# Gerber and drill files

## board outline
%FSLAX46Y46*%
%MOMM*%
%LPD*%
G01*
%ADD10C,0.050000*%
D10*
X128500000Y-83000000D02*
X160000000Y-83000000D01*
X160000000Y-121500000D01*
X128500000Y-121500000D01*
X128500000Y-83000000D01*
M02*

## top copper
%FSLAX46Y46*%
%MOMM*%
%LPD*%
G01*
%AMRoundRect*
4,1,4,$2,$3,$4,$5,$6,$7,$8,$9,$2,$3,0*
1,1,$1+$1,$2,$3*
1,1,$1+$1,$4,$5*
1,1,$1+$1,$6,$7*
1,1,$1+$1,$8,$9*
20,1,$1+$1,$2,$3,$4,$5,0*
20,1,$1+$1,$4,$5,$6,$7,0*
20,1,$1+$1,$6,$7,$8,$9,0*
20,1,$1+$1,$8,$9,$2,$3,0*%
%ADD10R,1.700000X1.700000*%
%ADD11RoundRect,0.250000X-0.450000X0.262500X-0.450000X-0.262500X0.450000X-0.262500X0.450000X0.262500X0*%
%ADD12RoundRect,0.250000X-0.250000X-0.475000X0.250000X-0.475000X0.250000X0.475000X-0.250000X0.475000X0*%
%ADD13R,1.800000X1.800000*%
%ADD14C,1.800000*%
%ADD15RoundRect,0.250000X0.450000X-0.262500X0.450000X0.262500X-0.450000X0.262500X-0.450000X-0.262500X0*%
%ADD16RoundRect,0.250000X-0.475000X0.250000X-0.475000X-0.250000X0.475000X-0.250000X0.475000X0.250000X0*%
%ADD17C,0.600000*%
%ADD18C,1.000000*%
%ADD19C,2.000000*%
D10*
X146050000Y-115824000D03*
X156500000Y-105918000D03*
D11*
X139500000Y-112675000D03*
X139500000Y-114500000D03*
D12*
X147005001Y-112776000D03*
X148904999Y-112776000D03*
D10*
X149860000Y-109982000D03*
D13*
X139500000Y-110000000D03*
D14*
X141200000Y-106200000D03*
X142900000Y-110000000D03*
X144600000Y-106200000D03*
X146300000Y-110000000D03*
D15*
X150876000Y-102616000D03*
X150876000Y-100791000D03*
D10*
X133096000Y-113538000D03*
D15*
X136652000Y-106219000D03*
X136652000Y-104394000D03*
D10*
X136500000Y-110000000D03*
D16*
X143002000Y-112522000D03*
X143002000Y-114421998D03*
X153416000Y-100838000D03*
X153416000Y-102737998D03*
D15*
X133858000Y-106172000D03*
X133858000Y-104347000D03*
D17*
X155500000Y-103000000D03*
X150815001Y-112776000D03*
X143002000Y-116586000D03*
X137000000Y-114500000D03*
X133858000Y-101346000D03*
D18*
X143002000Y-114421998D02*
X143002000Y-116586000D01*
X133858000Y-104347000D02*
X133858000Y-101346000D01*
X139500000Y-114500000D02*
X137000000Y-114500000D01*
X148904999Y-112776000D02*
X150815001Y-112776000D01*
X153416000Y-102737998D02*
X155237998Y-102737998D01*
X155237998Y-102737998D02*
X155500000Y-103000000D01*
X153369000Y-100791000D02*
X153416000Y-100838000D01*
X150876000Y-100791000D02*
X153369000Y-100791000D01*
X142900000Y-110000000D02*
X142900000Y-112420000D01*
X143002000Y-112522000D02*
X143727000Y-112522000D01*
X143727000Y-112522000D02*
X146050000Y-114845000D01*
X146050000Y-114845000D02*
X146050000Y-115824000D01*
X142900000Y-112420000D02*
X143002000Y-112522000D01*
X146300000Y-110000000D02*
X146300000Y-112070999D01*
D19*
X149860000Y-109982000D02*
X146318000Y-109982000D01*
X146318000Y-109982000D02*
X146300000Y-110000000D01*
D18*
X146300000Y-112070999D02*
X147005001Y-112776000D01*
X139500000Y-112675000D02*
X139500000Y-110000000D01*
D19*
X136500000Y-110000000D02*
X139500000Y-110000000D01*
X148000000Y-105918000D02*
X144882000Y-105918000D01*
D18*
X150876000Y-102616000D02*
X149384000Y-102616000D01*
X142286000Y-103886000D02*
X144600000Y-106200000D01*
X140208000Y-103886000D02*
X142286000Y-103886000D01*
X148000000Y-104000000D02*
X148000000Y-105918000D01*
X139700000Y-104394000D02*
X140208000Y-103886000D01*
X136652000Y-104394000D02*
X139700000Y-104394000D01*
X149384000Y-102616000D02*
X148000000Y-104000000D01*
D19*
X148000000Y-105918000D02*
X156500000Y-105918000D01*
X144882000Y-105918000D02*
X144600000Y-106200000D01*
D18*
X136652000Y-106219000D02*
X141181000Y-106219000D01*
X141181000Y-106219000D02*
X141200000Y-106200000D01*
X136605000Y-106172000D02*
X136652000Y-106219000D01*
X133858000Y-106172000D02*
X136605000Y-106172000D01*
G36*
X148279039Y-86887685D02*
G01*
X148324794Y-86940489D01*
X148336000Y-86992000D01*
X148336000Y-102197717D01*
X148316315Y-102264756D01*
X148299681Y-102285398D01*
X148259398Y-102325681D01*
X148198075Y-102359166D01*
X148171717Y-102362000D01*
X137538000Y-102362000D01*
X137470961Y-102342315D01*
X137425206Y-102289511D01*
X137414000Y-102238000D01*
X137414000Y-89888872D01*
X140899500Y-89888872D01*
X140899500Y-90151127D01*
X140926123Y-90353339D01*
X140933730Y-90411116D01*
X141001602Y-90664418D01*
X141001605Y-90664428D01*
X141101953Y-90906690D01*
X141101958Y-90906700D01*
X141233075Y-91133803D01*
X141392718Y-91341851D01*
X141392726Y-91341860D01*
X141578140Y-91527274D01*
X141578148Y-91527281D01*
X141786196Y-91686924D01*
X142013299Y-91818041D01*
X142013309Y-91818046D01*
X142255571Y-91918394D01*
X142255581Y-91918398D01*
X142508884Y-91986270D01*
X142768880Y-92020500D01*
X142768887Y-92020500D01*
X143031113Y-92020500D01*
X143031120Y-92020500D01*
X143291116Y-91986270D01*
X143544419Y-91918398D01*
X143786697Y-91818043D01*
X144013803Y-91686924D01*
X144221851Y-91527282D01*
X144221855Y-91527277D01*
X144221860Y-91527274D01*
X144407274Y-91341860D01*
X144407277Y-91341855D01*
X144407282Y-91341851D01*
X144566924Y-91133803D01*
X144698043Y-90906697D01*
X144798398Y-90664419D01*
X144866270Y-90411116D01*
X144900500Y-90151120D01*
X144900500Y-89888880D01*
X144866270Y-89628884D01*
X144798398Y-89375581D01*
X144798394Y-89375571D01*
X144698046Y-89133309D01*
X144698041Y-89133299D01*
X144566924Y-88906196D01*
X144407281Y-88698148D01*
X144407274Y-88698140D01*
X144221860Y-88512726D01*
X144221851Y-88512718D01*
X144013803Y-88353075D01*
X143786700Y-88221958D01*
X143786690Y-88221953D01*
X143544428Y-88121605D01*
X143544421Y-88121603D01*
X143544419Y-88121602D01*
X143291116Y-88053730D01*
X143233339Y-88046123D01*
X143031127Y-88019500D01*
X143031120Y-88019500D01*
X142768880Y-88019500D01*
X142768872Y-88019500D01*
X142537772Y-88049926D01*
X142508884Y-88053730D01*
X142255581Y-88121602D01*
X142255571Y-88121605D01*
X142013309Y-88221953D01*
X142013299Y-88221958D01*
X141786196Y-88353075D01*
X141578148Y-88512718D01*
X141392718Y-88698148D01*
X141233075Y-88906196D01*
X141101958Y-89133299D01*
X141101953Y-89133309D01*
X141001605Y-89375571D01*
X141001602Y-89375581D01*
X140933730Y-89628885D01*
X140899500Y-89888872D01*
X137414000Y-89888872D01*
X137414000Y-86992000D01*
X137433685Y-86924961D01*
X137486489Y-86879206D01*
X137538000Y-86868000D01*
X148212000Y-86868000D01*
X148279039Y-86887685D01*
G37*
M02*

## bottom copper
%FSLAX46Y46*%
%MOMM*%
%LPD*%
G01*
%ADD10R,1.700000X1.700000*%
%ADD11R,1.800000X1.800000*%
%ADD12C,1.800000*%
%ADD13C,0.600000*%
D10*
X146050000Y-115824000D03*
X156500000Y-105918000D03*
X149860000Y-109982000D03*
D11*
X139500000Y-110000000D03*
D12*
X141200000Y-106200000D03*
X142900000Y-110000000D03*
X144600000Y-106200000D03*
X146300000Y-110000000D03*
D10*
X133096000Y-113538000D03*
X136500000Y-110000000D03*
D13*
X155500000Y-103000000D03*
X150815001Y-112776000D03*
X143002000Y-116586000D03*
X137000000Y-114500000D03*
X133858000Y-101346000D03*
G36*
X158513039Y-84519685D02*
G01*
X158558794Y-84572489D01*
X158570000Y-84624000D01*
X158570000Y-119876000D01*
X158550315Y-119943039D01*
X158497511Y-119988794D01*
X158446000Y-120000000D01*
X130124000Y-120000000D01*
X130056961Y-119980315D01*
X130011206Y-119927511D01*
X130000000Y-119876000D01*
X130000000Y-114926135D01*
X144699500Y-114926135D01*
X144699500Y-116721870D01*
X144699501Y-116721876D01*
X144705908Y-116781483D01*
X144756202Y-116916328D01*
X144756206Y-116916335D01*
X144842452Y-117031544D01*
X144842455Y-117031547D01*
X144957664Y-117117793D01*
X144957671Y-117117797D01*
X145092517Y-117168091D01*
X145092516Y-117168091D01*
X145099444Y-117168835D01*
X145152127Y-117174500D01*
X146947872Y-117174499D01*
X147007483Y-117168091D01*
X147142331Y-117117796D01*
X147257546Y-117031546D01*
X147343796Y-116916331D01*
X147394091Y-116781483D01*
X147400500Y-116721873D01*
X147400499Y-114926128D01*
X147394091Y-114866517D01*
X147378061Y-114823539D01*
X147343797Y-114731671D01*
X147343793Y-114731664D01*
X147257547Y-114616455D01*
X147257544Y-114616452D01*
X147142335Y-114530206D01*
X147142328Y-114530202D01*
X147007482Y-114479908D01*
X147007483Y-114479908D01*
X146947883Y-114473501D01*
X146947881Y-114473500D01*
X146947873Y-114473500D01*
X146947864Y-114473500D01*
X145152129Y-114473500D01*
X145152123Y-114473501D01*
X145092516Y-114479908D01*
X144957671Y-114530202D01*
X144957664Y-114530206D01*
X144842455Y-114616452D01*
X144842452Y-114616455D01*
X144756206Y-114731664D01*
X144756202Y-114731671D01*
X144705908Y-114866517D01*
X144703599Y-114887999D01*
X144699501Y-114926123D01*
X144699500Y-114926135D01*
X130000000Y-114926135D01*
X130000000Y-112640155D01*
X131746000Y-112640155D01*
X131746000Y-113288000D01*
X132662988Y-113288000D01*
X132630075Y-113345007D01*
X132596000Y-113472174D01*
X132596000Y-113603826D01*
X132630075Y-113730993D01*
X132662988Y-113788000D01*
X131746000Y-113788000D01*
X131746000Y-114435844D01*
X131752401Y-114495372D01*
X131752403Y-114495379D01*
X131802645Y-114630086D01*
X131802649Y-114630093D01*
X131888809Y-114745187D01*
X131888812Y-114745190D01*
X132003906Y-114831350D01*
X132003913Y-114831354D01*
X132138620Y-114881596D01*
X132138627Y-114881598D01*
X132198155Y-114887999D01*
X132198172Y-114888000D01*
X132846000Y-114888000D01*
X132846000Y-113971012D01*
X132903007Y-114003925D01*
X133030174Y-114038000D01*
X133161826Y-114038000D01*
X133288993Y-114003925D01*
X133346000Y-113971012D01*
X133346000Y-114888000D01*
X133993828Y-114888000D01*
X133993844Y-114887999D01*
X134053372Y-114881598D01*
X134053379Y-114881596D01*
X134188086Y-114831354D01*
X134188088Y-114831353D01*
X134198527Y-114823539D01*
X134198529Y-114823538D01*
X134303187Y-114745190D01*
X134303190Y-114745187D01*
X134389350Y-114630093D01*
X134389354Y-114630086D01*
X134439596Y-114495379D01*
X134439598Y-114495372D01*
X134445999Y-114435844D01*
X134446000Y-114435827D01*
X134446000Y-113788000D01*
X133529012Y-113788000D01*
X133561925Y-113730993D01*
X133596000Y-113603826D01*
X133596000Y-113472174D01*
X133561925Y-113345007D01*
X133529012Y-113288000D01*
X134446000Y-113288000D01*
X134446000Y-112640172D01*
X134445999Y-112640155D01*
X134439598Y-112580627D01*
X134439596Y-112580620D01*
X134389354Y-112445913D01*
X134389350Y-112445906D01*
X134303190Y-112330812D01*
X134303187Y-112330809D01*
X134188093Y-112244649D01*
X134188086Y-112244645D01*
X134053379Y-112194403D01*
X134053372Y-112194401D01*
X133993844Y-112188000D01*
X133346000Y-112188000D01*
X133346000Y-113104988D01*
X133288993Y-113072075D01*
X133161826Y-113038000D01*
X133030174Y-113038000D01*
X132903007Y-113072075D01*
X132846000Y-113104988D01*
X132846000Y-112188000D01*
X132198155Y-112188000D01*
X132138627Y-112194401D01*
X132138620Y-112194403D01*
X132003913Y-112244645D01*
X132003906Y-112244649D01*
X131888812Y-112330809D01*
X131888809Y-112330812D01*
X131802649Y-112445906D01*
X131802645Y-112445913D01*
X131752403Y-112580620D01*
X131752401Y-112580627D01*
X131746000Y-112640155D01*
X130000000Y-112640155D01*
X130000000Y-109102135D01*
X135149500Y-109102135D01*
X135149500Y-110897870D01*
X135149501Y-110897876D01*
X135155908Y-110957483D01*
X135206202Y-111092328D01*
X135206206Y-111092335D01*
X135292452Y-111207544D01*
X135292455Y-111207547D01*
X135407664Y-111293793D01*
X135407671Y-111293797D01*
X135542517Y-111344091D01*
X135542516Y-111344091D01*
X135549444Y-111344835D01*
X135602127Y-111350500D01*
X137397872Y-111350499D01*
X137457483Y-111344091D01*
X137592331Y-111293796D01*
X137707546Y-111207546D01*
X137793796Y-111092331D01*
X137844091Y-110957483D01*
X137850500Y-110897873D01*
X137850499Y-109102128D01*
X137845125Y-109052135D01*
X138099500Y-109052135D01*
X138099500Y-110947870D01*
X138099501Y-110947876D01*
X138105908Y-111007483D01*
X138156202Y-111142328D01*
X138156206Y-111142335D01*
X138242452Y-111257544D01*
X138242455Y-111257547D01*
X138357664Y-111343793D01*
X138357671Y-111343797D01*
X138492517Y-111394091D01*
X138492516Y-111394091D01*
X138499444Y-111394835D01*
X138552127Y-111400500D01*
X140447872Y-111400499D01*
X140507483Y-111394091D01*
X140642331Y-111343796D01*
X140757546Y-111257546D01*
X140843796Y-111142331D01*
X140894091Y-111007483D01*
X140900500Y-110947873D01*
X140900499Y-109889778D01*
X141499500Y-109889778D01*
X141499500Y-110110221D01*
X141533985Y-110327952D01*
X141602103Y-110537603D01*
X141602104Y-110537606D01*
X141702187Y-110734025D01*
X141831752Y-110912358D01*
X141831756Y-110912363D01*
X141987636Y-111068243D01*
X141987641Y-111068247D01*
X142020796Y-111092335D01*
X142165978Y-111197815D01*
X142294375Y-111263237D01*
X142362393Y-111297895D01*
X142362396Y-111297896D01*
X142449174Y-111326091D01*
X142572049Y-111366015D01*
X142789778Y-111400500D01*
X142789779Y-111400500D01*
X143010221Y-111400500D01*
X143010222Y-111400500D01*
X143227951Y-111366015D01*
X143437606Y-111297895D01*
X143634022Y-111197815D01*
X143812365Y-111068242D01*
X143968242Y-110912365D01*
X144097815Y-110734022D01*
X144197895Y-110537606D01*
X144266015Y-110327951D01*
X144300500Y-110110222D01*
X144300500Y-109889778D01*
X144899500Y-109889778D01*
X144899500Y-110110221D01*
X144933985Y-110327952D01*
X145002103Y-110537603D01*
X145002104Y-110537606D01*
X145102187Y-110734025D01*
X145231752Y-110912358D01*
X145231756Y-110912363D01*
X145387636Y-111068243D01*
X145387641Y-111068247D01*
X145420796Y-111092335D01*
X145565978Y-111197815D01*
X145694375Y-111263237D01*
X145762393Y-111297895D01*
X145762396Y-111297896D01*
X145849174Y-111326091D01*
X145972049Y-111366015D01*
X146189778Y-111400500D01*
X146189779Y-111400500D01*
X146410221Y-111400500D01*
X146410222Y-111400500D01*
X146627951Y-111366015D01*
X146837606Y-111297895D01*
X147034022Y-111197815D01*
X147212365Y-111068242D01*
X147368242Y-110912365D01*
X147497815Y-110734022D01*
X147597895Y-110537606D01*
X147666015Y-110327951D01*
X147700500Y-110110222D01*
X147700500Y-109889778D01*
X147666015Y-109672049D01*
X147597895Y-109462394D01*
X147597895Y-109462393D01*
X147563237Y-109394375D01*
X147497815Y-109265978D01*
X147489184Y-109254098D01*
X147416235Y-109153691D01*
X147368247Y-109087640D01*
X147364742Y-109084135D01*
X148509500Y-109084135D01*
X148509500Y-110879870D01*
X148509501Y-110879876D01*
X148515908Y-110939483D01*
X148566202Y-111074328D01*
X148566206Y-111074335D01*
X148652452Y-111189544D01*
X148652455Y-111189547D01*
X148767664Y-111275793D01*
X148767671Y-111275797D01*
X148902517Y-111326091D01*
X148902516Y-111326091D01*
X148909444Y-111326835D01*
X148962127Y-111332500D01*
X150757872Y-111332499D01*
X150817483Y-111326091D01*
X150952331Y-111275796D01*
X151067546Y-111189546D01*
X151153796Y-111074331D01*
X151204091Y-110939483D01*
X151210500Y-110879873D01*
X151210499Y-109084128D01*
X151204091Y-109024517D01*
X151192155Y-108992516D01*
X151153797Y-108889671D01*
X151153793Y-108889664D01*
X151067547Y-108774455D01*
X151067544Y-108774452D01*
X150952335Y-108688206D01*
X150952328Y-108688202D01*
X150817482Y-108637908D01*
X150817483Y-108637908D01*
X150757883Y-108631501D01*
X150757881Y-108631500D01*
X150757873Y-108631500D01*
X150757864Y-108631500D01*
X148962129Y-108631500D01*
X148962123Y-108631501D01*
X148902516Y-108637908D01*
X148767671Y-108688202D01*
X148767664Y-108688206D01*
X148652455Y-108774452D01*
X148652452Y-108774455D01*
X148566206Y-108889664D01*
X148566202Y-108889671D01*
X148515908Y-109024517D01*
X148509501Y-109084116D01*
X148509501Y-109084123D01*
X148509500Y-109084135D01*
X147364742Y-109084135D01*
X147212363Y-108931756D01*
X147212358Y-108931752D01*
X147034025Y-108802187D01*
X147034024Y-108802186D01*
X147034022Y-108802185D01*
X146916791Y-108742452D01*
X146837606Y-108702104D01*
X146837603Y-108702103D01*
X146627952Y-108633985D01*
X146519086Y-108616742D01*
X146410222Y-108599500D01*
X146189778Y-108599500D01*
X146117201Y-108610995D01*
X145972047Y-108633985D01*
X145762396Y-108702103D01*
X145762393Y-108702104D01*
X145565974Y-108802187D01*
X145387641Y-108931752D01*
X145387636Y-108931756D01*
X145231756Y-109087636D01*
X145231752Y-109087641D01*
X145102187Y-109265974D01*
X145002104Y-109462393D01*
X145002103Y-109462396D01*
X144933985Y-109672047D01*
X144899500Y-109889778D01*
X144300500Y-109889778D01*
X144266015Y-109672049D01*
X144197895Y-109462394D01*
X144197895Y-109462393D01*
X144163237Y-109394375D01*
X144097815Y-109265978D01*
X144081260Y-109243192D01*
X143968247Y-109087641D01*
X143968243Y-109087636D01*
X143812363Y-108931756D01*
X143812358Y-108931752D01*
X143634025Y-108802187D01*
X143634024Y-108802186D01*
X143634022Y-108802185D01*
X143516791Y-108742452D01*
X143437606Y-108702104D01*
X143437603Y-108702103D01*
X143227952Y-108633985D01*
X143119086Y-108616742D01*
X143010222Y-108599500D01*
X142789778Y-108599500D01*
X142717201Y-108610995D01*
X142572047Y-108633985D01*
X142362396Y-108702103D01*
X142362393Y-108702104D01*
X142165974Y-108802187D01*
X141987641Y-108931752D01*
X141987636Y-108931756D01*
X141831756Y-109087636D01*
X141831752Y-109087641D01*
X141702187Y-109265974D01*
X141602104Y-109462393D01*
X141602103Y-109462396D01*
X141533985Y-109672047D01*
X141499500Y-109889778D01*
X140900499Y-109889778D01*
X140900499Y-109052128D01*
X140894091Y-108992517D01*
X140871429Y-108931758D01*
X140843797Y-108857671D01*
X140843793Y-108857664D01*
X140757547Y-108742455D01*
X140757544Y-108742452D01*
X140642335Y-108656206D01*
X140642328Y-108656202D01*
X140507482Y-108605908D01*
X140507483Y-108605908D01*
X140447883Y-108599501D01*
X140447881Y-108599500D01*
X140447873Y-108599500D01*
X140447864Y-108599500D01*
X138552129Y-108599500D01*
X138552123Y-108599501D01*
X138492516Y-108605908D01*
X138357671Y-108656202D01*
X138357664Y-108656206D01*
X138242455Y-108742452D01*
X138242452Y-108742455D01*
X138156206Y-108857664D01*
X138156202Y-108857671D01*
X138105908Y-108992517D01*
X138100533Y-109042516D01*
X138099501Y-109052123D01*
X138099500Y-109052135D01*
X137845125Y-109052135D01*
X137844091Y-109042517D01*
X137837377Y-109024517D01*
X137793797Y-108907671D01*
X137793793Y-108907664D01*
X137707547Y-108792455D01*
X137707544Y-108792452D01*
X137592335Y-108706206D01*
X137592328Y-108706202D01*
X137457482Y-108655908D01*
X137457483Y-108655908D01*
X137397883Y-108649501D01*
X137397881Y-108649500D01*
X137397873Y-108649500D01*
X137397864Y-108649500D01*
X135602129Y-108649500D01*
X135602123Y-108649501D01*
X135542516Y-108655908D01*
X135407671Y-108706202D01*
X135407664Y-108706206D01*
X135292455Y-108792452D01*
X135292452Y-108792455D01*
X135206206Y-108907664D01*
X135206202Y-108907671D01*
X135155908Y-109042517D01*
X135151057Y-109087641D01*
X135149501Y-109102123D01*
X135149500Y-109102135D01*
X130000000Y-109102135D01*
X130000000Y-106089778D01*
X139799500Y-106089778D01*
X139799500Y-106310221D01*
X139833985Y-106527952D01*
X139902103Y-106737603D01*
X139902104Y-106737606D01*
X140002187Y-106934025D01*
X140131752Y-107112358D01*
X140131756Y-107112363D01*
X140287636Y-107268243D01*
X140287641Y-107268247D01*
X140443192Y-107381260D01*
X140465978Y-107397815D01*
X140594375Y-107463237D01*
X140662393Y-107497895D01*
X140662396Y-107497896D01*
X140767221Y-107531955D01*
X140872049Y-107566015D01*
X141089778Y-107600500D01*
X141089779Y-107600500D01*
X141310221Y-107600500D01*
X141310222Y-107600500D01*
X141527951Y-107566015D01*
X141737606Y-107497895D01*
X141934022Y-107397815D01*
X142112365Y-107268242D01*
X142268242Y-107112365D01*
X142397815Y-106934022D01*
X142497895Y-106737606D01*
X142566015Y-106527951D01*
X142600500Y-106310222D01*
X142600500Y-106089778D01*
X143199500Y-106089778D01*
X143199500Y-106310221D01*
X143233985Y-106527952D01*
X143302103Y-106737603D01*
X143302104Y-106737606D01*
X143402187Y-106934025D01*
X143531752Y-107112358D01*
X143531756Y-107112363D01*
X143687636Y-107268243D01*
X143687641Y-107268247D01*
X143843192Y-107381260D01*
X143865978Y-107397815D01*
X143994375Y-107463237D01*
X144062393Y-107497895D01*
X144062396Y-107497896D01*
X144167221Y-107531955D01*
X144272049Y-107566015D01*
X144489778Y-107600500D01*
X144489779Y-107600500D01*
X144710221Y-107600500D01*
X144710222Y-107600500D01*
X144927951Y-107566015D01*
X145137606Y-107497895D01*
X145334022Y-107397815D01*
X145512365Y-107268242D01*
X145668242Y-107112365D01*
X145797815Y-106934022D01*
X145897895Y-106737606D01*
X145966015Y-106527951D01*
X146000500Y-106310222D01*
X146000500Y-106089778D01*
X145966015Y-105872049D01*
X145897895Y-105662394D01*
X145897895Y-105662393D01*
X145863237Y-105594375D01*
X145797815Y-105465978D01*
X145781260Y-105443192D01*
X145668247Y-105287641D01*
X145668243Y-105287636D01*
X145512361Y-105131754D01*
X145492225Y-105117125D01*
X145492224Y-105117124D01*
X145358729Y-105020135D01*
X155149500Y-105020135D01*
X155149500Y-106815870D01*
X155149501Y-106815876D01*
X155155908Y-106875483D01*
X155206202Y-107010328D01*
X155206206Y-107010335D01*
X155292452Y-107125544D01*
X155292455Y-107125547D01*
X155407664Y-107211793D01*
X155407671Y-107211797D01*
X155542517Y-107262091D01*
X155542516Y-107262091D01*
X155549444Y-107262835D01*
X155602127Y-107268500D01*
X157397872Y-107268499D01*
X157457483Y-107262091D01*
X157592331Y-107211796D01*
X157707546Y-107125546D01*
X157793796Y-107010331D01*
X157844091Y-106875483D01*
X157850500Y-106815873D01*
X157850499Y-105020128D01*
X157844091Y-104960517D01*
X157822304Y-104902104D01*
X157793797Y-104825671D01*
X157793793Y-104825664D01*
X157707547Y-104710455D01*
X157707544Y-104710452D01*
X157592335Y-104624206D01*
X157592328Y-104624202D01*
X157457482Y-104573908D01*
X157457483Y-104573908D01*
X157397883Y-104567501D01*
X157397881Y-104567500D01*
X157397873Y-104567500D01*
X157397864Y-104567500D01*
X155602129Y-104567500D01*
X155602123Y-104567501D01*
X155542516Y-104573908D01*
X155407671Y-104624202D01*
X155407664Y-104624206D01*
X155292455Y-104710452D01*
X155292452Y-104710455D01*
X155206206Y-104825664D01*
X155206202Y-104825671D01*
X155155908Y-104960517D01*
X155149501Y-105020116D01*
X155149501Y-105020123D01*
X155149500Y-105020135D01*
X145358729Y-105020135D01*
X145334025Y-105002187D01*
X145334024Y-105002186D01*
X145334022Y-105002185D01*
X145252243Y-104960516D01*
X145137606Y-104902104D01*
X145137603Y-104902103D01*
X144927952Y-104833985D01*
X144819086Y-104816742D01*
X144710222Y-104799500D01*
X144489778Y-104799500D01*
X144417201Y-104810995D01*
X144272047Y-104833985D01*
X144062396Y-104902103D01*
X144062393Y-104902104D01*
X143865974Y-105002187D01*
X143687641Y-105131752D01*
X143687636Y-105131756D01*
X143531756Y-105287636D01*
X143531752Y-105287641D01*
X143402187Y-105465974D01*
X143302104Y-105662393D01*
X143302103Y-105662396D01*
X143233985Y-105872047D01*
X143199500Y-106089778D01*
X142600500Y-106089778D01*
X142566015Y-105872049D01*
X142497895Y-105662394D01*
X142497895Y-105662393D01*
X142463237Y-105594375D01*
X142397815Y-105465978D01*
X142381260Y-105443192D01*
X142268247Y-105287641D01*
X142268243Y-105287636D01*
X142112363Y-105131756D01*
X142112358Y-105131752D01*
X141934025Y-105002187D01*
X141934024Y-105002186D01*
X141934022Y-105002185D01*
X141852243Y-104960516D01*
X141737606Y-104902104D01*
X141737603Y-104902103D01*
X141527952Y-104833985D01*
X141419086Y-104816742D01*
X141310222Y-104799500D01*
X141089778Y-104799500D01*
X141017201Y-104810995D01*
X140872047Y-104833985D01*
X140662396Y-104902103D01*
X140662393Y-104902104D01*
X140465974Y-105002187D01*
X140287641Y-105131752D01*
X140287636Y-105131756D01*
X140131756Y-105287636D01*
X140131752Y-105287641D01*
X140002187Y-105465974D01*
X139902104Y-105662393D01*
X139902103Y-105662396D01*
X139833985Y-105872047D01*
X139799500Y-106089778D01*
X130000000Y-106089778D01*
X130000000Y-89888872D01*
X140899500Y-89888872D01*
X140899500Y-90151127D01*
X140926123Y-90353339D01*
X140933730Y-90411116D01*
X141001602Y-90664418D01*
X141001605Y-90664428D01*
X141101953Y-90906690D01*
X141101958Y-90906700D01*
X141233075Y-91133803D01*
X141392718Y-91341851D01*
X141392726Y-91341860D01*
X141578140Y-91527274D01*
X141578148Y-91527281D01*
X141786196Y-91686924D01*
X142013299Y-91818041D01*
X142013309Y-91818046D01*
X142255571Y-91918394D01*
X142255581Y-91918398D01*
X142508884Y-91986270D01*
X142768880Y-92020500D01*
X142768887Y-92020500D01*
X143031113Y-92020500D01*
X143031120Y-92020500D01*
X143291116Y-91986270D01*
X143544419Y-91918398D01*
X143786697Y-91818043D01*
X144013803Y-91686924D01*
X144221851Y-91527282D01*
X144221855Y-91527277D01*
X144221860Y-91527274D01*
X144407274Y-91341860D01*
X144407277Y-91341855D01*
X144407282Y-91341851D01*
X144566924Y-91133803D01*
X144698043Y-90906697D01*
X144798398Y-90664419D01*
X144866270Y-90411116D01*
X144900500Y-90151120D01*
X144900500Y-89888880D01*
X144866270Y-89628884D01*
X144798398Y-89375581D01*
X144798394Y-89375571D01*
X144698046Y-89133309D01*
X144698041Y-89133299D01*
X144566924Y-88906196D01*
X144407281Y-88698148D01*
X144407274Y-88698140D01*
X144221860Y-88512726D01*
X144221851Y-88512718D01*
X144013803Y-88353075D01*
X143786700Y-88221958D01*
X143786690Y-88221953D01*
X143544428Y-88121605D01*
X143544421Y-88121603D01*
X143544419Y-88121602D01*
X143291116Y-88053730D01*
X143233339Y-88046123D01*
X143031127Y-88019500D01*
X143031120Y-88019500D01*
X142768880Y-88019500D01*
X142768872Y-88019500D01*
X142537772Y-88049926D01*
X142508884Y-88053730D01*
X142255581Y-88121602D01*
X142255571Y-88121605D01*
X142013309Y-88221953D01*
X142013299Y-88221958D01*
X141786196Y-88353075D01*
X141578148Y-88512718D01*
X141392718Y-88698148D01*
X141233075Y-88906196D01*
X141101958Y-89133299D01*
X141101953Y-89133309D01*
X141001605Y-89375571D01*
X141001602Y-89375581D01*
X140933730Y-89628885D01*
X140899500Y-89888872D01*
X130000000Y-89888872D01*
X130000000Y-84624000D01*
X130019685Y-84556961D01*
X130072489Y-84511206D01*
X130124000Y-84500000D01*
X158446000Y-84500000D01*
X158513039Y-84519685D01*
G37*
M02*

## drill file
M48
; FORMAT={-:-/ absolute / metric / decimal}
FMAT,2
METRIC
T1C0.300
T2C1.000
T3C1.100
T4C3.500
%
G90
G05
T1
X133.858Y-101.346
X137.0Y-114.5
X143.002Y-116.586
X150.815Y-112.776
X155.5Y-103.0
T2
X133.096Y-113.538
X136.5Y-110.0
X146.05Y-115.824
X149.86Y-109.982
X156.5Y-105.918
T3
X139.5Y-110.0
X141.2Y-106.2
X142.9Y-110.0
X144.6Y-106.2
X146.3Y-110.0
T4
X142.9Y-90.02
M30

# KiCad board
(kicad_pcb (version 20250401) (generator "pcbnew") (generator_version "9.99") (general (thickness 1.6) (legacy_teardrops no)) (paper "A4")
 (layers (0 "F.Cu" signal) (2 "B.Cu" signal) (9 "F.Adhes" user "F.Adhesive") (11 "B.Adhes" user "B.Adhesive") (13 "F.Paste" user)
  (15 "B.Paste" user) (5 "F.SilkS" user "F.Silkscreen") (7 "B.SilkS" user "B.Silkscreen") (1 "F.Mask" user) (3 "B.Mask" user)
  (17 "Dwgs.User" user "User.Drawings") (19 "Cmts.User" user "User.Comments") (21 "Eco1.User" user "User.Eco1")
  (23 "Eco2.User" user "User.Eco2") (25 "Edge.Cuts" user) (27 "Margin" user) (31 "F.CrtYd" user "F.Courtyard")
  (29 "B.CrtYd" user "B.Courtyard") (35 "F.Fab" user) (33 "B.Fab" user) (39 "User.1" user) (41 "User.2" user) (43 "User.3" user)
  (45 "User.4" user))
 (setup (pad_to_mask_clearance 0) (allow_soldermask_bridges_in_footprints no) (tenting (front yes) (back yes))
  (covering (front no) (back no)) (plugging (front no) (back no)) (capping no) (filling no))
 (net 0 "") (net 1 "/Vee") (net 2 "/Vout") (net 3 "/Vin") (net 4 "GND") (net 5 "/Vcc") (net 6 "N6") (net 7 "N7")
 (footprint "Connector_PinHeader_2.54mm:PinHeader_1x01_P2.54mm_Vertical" (layer "F.Cu") (at 146.05 115.824)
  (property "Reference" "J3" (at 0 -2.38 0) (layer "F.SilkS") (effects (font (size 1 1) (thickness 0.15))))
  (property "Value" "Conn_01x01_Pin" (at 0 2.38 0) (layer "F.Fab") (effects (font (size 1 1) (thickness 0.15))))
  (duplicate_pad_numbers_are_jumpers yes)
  (pad "1" thru_hole rect (at 0 0) (size 1.7 1.7) (drill 1) (layers "*.Cu" "*.Mask") (remove_unused_layers no) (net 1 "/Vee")
   (tenting (front none) (back none))))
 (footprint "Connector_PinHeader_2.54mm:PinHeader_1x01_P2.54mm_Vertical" (layer "F.Cu") (at 156.5 105.918)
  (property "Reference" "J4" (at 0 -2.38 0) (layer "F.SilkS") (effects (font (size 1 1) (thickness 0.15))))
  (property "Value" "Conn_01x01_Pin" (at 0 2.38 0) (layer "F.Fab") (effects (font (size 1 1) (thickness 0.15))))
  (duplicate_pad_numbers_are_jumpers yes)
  (pad "1" thru_hole rect (at 0 0) (size 1.7 1.7) (drill 1) (layers "*.Cu" "*.Mask") (remove_unused_layers no) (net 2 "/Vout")
   (tenting (front none) (back none))))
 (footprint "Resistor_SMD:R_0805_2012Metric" (layer "F.Cu") (at 139.5 113.5875 -90)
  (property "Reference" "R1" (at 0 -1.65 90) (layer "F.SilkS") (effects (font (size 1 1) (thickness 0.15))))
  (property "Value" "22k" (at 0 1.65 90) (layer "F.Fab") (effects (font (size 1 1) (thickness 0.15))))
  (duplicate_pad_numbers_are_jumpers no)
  (pad "1" smd roundrect (at -0.9125 0 270) (size 1.025 1.4) (layers "F.Cu" "F.Mask" "F.Paste") (roundrect_rratio 0.243902) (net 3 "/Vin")
   (tenting (front none) (back none)))
  (pad "2" smd roundrect (at 0.9125 0 270) (size 1.025 1.4) (layers "F.Cu" "F.Mask" "F.Paste") (roundrect_rratio 0.243902) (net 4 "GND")
   (tenting (front none) (back none))))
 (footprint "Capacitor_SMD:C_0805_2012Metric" (layer "F.Cu") (at 147.955 112.776)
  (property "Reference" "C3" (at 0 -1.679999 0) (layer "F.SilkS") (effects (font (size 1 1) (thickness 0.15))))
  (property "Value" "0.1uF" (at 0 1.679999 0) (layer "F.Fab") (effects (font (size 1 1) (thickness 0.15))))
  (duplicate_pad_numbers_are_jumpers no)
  (pad "1" smd roundrect (at -0.949999 0) (size 1 1.45) (layers "F.Cu" "F.Mask" "F.Paste") (roundrect_rratio 0.25) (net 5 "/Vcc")
   (tenting (front none) (back none)))
  (pad "2" smd roundrect (at 0.949999 0) (size 1 1.45) (layers "F.Cu" "F.Mask" "F.Paste") (roundrect_rratio 0.25) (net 4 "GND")
   (tenting (front none) (back none))))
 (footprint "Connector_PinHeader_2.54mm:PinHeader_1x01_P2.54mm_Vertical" (layer "F.Cu") (at 149.86 109.982)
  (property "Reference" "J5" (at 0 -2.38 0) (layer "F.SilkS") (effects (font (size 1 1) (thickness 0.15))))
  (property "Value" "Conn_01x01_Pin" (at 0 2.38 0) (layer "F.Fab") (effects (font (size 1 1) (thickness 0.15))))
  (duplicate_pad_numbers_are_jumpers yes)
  (pad "1" thru_hole rect (at 0 0) (size 1.7 1.7) (drill 1) (layers "*.Cu" "*.Mask") (remove_unused_layers no) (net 5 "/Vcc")
   (tenting (front none) (back none))))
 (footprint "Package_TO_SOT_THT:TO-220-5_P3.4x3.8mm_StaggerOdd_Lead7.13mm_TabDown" (layer "F.Cu") (at 139.5 110)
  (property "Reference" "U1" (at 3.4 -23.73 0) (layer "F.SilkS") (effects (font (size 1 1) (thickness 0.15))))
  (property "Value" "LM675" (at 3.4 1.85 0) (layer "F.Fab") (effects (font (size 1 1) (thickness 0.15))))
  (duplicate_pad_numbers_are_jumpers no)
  (pad "" np_thru_hole circle (at 3.4 -19.98) (size 3.5 3.5) (drill 3.5) (layers "*.Cu" "*.Mask") (tenting (front none) (back none)))
  (pad "1" thru_hole rect (at 0 0) (size 1.8 1.8) (drill 1.1) (layers "*.Cu" "*.Mask") (remove_unused_layers no) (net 3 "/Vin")
   (tenting (front none) (back none)))
  (pad "2" thru_hole circle (at 1.7 -3.8) (size 1.8 1.8) (drill 1.1) (layers "*.Cu" "*.Mask") (remove_unused_layers no) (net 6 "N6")
   (tenting (front none) (back none)))
  (pad "3" thru_hole circle (at 3.4 0) (size 1.8 1.8) (drill 1.1) (layers "*.Cu" "*.Mask") (remove_unused_layers no) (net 1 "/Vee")
   (tenting (front none) (back none)))
  (pad "4" thru_hole circle (at 5.1 -3.8) (size 1.8 1.8) (drill 1.1) (layers "*.Cu" "*.Mask") (remove_unused_layers no) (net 2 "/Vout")
   (tenting (front none) (back none)))
  (pad "5" thru_hole circle (at 6.8 0) (size 1.8 1.8) (drill 1.1) (layers "*.Cu" "*.Mask") (remove_unused_layers no) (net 5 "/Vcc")
   (tenting (front none) (back none))))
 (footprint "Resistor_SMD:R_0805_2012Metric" (layer "F.Cu") (at 150.876 101.7035 90)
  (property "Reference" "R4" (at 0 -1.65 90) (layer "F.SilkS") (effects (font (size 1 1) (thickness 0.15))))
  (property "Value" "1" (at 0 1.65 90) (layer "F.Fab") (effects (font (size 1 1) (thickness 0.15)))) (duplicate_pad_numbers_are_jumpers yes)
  (pad "1" smd roundrect (at -0.9125 0 90) (size 1.025 1.4) (layers "F.Cu" "F.Mask" "F.Paste") (roundrect_rratio 0.243902) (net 2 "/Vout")
   (tenting (front none) (back none)))
  (pad "2" smd roundrect (at 0.9125 0 90) (size 1.025 1.4) (layers "F.Cu" "F.Mask" "F.Paste") (roundrect_rratio 0.243902) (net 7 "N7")
   (tenting (front none) (back none))))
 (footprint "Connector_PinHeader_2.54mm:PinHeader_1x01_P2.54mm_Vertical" (layer "F.Cu") (at 133.096 113.538)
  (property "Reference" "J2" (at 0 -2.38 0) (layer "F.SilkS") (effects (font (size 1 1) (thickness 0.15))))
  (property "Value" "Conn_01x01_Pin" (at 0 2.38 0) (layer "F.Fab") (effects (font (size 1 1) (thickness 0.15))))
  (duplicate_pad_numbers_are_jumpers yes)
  (pad "1" thru_hole rect (at 0 0) (size 1.7 1.7) (drill 1) (layers "*.Cu" "*.Mask") (remove_unused_layers no) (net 4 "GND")
   (tenting (front none) (back none))))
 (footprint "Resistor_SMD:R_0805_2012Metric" (layer "F.Cu") (at 136.652 105.3065 90)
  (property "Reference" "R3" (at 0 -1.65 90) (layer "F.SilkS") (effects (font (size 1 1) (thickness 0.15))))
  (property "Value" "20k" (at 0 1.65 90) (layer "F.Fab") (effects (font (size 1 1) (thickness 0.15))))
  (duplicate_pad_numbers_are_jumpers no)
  (pad "1" smd roundrect (at -0.9125 0 90) (size 1.025 1.4) (layers "F.Cu" "F.Mask" "F.Paste") (roundrect_rratio 0.243902) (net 6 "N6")
   (tenting (front none) (back none)))
  (pad "2" smd roundrect (at 0.9125 0 90) (size 1.025 1.4) (layers "F.Cu" "F.Mask" "F.Paste") (roundrect_rratio 0.243902) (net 2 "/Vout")
   (tenting (front none) (back none))))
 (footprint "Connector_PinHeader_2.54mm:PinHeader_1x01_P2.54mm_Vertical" (layer "F.Cu") (at 136.5 110)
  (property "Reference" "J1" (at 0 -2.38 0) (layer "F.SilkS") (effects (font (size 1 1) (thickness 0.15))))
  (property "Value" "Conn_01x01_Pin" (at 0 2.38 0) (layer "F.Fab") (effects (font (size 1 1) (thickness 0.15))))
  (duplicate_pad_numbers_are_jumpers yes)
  (pad "1" thru_hole rect (at 0 0) (size 1.7 1.7) (drill 1) (layers "*.Cu" "*.Mask") (remove_unused_layers no) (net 3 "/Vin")
   (tenting (front none) (back none))))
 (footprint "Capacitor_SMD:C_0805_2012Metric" (layer "F.Cu") (at 143.002 113.471999 -90)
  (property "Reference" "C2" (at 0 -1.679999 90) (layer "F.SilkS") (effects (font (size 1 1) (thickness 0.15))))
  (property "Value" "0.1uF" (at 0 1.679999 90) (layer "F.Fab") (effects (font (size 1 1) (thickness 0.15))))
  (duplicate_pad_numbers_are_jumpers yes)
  (pad "1" smd roundrect (at -0.949999 0 270) (size 1 1.45) (layers "F.Cu" "F.Mask" "F.Paste") (roundrect_rratio 0.25) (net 1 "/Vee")
   (tenting (front none) (back none)))
  (pad "2" smd roundrect (at 0.949999 0 270) (size 1 1.45) (layers "F.Cu" "F.Mask" "F.Paste") (roundrect_rratio 0.25) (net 4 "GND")
   (tenting (front none) (back none))))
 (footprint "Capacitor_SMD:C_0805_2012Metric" (layer "F.Cu") (at 153.416 101.787999 -90)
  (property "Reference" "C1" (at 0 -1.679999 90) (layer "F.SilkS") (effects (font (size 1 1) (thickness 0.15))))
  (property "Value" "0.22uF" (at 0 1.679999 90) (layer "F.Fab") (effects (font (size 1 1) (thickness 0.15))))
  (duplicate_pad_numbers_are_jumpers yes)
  (pad "1" smd roundrect (at -0.949999 0 270) (size 1 1.45) (layers "F.Cu" "F.Mask" "F.Paste") (roundrect_rratio 0.25) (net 7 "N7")
   (tenting (front none) (back none)))
  (pad "2" smd roundrect (at 0.949999 0 270) (size 1 1.45) (layers "F.Cu" "F.Mask" "F.Paste") (roundrect_rratio 0.25) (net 4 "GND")
   (tenting (front none) (back none))))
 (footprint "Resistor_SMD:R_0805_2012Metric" (layer "F.Cu") (at 133.858 105.2595 90)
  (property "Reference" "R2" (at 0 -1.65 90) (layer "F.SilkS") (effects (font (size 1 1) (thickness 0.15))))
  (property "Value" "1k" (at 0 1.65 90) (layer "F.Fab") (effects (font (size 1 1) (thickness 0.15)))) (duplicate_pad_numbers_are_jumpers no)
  (pad "1" smd roundrect (at -0.9125 0 90) (size 1.025 1.4) (layers "F.Cu" "F.Mask" "F.Paste") (roundrect_rratio 0.243902) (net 6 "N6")
   (tenting (front none) (back none)))
  (pad "2" smd roundrect (at 0.9125 0 90) (size 1.025 1.4) (layers "F.Cu" "F.Mask" "F.Paste") (roundrect_rratio 0.243902) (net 4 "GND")
   (tenting (front none) (back none))))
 (gr_rect (start 128.5 83) (end 160 121.5) (stroke (width 0.05) (type default)) (fill no) (layer "Edge.Cuts"))
 (segment (start 143.002 114.421998) (end 143.002 116.586) (width 1) (layer "F.Cu") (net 4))
 (segment (start 133.858 104.347) (end 133.858 101.346) (width 1) (layer "F.Cu") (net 4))
 (segment (start 139.5 114.5) (end 137 114.5) (width 1) (layer "F.Cu") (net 4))
 (segment (start 148.904999 112.776) (end 150.815001 112.776) (width 1) (layer "F.Cu") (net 4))
 (segment (start 153.416 102.737998) (end 155.237998 102.737998) (width 1) (layer "F.Cu") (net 4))
 (segment (start 155.237998 102.737998) (end 155.5 103) (width 1) (layer "F.Cu") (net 4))
 (via (at 155.5 103) (size 0.6) (drill 0.3) (layers "F.Cu" "B.Cu") (tenting (front none) (back none)) (capping none)
  (covering (front none) (back none)) (plugging (front none) (back none)) (filling none) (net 4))
 (via (at 150.815001 112.776) (size 0.6) (drill 0.3) (layers "F.Cu" "B.Cu") (tenting (front none) (back none)) (capping none)
  (covering (front none) (back none)) (plugging (front none) (back none)) (filling none) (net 4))
 (via (at 143.002 116.586) (size 0.6) (drill 0.3) (layers "F.Cu" "B.Cu") (tenting (front none) (back none)) (capping none)
  (covering (front none) (back none)) (plugging (front none) (back none)) (filling none) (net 4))
 (via (at 137 114.5) (size 0.6) (drill 0.3) (layers "F.Cu" "B.Cu") (tenting (front none) (back none)) (capping none)
  (covering (front none) (back none)) (plugging (front none) (back none)) (filling none) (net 4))
 (via (at 133.858 101.346) (size 0.6) (drill 0.3) (layers "F.Cu" "B.Cu") (tenting (front none) (back none)) (capping none)
  (covering (front none) (back none)) (plugging (front none) (back none)) (filling none) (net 4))
 (segment (start 153.369 100.791) (end 153.416 100.838) (width 1) (layer "F.Cu") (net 7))
 (segment (start 150.876 100.791) (end 153.369 100.791) (width 1) (layer "F.Cu") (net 7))
 (segment (start 142.9 110) (end 142.9 112.42) (width 1) (layer "F.Cu") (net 1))
 (segment (start 143.002 112.522) (end 143.727 112.522) (width 1) (layer "F.Cu") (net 1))
 (segment (start 143.727 112.522) (end 146.05 114.845) (width 1) (layer "F.Cu") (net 1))
 (segment (start 146.05 114.845) (end 146.05 115.824) (width 1) (layer "F.Cu") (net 1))
 (segment (start 142.9 112.42) (end 143.002 112.522) (width 1) (layer "F.Cu") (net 1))
 (segment (start 146.3 110) (end 146.3 112.070999) (width 1) (layer "F.Cu") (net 5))
 (segment (start 149.86 109.982) (end 146.318 109.982) (width 2) (layer "F.Cu") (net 5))
 (segment (start 146.318 109.982) (end 146.3 110) (width 2) (layer "F.Cu") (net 5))
 (segment (start 146.3 112.070999) (end 147.005001 112.776) (width 1) (layer "F.Cu") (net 5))
 (segment (start 139.5 112.675) (end 139.5 110) (width 1) (layer "F.Cu") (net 3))
 (segment (start 136.5 110) (end 139.5 110) (width 2) (layer "F.Cu") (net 3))
 (segment (start 148 105.918) (end 144.882 105.918) (width 2) (layer "F.Cu") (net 2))
 (segment (start 150.876 102.616) (end 149.384 102.616) (width 1) (layer "F.Cu") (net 2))
 (segment (start 142.286 103.886) (end 144.6 106.2) (width 1) (layer "F.Cu") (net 2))
 (segment (start 140.208 103.886) (end 142.286 103.886) (width 1) (layer "F.Cu") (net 2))
 (segment (start 148 104) (end 148 105.918) (width 1) (layer "F.Cu") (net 2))
 (segment (start 139.7 104.394) (end 140.208 103.886) (width 1) (layer "F.Cu") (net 2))
 (segment (start 136.652 104.394) (end 139.7 104.394) (width 1) (layer "F.Cu") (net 2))
 (segment (start 149.384 102.616) (end 148 104) (width 1) (layer "F.Cu") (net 2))
 (segment (start 148 105.918) (end 156.5 105.918) (width 2) (layer "F.Cu") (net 2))
 (segment (start 144.882 105.918) (end 144.6 106.2) (width 2) (layer "F.Cu") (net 2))
 (segment (start 136.652 106.219) (end 141.181 106.219) (width 1) (layer "F.Cu") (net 6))
 (segment (start 141.181 106.219) (end 141.2 106.2) (width 1) (layer "F.Cu") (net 6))
 (segment (start 136.605 106.172) (end 136.652 106.219) (width 1) (layer "F.Cu") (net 6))
 (segment (start 133.858 106.172) (end 136.605 106.172) (width 1) (layer "F.Cu") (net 6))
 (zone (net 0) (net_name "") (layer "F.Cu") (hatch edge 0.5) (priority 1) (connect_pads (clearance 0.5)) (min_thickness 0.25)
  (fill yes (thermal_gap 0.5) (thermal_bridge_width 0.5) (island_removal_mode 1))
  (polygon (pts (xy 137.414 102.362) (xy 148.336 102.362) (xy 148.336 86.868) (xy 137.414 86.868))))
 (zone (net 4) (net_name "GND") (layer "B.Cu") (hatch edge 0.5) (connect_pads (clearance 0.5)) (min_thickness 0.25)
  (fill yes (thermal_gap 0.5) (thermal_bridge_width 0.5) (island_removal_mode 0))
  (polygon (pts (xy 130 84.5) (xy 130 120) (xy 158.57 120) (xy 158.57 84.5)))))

